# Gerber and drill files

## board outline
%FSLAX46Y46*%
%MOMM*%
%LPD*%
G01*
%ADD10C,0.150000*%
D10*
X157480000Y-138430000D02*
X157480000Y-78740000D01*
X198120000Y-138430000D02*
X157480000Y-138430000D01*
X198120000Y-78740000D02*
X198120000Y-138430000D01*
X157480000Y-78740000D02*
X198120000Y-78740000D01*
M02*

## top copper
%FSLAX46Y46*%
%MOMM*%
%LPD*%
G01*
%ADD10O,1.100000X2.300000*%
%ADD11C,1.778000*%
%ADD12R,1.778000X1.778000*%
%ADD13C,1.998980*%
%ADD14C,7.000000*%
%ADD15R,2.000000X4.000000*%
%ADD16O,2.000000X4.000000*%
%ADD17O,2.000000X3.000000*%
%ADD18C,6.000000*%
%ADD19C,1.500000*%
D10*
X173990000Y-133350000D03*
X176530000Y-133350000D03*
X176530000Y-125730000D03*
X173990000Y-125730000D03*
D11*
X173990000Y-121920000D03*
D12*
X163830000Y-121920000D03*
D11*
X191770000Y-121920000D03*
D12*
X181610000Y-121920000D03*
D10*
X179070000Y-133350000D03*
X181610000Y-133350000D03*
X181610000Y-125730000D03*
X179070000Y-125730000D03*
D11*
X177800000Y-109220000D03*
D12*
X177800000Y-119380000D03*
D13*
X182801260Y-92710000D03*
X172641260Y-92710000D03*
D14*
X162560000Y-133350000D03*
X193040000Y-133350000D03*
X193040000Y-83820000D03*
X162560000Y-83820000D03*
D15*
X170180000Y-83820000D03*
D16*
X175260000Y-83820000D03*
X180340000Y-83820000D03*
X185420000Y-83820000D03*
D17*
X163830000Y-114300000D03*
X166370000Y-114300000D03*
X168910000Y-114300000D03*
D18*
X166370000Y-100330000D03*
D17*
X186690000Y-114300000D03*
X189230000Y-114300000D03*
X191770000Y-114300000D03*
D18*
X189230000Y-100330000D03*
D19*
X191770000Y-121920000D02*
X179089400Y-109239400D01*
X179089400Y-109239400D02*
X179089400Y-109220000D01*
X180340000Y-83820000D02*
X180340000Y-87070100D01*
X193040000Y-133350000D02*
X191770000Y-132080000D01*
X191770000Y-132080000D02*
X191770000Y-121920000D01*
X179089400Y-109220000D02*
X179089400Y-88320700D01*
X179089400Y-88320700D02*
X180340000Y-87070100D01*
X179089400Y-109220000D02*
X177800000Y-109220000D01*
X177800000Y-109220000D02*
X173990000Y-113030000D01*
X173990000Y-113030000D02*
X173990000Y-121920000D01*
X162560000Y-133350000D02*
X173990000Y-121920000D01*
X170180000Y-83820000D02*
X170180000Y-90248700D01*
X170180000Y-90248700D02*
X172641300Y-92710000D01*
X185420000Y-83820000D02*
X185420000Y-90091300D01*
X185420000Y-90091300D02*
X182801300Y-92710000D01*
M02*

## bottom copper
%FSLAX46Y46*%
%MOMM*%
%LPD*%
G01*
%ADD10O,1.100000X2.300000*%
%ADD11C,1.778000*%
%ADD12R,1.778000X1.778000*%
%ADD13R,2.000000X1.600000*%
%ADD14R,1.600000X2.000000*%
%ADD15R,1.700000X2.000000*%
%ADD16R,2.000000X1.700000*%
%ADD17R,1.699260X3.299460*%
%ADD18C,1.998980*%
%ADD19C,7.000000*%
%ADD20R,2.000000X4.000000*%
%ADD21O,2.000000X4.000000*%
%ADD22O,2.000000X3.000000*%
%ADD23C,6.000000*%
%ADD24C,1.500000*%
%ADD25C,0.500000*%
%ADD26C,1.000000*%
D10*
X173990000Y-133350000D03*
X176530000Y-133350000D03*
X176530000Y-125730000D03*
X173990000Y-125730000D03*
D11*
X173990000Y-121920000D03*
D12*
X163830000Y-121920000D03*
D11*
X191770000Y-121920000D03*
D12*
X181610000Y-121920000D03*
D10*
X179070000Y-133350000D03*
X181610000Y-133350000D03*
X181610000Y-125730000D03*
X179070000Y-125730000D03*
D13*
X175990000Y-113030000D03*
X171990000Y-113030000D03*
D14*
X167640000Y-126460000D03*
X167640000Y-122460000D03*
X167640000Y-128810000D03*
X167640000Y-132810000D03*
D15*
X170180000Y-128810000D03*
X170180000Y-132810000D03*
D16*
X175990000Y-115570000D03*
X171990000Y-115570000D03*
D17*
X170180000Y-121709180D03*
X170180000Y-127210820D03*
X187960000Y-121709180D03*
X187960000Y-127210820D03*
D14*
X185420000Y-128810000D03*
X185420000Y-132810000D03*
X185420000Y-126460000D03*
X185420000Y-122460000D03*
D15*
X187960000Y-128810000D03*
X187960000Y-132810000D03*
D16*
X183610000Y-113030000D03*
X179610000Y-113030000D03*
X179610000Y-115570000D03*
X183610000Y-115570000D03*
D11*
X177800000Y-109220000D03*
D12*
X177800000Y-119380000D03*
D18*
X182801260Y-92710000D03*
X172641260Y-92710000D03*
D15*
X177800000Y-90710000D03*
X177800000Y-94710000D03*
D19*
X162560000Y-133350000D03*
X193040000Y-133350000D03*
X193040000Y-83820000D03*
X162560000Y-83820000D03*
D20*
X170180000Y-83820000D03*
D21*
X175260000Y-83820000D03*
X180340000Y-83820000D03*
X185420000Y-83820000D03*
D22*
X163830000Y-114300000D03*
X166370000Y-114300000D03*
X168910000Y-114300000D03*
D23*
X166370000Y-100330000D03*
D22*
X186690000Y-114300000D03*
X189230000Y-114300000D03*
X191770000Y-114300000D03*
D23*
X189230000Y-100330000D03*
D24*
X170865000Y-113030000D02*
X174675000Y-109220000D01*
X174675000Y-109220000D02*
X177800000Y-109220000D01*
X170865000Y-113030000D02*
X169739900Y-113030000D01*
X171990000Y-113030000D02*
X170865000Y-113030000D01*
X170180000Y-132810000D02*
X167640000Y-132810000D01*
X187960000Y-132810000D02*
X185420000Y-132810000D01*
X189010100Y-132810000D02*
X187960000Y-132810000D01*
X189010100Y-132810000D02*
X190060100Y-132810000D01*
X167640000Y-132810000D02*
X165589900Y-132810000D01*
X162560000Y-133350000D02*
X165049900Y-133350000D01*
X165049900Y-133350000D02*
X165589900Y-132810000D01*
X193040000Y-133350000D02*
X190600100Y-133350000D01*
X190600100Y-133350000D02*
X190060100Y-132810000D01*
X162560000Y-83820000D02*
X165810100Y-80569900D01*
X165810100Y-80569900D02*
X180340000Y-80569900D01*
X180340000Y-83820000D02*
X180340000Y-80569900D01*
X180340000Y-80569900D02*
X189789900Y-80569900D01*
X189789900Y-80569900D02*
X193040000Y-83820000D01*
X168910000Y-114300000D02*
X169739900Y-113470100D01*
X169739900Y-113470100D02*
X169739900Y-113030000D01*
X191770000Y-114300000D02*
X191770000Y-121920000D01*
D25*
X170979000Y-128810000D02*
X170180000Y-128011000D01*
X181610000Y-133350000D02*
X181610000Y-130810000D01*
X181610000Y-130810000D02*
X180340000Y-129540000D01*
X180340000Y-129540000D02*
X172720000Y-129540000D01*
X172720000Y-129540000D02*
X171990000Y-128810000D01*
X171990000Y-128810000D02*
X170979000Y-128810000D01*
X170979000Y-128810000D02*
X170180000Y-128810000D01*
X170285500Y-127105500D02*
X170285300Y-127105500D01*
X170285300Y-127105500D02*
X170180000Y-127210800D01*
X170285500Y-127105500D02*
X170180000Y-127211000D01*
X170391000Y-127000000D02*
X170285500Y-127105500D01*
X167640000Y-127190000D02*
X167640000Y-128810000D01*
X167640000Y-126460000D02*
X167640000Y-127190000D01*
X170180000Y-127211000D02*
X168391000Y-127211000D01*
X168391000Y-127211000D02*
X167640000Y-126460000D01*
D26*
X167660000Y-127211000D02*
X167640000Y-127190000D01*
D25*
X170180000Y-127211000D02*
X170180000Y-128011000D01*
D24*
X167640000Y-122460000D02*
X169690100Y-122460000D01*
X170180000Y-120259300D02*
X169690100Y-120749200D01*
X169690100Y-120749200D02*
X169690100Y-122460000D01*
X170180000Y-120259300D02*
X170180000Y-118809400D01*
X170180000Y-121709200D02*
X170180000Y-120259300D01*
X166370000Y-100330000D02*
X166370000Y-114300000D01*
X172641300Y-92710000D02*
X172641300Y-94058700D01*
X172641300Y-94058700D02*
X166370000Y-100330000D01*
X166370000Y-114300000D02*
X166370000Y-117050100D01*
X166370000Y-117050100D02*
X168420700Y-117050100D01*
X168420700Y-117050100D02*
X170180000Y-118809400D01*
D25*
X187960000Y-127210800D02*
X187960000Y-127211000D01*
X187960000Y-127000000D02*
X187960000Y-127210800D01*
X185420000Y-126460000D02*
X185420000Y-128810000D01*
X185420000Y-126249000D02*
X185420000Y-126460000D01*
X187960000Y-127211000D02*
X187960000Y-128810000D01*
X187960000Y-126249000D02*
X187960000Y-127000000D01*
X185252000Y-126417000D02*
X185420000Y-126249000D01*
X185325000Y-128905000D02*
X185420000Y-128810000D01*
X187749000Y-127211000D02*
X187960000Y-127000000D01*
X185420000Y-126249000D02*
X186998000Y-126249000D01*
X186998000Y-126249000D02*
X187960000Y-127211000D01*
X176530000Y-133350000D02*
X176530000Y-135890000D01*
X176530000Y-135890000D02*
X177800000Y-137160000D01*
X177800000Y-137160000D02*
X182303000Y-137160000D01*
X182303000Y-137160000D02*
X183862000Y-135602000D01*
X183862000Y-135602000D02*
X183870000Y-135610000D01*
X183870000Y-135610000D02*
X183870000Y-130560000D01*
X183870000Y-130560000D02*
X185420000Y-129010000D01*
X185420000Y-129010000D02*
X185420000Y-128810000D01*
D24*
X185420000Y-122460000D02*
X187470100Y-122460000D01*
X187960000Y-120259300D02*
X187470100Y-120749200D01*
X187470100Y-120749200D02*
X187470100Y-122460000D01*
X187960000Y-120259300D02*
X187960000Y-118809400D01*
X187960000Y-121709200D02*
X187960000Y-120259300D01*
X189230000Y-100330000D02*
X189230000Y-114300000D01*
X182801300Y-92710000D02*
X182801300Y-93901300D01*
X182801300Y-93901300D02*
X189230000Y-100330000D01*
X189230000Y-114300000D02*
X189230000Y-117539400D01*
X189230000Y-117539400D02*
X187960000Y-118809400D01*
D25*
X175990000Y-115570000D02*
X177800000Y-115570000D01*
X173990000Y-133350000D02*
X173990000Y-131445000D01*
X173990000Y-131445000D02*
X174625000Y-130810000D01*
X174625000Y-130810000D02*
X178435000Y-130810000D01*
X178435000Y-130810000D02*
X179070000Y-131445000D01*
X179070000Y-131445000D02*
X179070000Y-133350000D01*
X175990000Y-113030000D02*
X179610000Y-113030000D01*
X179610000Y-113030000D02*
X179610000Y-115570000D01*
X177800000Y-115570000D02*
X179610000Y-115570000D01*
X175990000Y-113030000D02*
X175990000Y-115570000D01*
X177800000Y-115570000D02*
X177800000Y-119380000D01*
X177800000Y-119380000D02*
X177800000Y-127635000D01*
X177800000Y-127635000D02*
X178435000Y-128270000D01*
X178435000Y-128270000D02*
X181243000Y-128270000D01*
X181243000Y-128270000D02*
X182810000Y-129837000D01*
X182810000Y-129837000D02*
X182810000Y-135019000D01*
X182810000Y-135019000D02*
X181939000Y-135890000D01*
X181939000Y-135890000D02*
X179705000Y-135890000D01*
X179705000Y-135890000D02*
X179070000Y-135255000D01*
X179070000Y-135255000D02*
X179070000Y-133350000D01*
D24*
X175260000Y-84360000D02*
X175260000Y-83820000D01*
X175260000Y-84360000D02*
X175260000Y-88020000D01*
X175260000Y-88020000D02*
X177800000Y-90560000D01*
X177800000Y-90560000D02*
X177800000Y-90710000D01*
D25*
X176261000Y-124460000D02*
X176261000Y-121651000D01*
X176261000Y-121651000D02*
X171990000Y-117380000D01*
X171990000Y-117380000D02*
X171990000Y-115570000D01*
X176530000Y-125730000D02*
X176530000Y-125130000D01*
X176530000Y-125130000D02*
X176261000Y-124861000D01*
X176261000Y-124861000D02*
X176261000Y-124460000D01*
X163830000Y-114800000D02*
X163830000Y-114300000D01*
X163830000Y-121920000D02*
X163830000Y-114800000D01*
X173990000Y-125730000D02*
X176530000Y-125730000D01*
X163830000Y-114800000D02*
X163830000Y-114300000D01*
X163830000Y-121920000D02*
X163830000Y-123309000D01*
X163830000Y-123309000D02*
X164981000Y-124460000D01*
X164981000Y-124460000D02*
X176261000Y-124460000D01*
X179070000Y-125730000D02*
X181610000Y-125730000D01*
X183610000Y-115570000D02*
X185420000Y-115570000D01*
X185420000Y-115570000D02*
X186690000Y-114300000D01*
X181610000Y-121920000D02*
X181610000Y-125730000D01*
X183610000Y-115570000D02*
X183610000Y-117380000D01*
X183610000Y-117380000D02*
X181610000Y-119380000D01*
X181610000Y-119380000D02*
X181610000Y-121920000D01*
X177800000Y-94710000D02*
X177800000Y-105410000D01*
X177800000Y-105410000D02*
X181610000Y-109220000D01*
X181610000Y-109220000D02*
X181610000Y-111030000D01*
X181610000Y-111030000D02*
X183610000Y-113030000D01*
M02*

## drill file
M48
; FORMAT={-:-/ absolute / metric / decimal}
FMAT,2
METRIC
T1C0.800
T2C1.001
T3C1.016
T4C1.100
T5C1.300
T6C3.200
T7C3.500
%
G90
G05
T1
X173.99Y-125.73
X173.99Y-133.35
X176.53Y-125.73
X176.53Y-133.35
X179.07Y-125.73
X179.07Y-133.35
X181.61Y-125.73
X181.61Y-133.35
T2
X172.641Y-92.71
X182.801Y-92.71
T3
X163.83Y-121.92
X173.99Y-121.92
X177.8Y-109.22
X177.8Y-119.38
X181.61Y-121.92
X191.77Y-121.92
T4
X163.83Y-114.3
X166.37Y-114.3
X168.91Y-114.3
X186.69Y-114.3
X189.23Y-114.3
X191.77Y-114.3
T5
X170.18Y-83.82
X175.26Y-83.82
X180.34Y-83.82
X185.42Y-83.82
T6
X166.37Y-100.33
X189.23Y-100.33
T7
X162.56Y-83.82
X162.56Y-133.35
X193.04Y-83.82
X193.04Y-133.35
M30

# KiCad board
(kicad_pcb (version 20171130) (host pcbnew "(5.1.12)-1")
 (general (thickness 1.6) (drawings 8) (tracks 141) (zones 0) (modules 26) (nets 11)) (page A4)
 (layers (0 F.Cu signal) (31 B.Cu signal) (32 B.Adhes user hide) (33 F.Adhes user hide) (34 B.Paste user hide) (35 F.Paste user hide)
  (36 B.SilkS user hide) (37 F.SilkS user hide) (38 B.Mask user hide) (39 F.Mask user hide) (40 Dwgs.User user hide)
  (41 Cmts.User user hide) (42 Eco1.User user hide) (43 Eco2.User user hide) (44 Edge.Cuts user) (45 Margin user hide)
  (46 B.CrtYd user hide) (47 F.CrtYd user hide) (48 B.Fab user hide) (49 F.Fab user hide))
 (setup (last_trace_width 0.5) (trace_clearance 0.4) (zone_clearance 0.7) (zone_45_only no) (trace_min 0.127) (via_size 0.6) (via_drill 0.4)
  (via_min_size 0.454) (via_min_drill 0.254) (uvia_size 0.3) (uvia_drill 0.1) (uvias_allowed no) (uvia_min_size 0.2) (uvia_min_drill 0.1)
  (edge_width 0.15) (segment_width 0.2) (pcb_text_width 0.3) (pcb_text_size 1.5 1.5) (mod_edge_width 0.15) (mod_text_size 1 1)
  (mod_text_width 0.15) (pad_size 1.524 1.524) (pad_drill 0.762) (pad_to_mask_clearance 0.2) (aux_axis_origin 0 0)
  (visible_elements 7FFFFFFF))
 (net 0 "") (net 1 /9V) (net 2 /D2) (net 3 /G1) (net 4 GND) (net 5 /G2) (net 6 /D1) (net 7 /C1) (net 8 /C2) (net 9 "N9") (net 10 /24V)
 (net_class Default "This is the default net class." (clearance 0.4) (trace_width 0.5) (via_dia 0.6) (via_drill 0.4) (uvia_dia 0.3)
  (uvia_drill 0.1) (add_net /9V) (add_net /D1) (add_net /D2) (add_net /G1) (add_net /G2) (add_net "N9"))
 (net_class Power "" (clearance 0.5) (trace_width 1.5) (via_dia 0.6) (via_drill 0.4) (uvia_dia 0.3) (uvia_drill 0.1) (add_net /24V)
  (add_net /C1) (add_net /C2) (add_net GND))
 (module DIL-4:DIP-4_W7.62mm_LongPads (layer F.Cu) (at 173.99 133.35 90)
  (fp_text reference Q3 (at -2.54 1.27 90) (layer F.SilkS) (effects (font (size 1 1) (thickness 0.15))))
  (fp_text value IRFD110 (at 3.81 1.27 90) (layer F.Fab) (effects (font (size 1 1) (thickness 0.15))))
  (pad 1 thru_hole oval (at 0 0 90) (size 2.3 1.1) (drill 0.8) (layers *.Cu *.Mask) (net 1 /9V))
  (pad 2 thru_hole oval (at 0 2.54 90) (size 2.3 1.1) (drill 0.8) (layers *.Cu *.Mask) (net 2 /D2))
  (pad 3 thru_hole oval (at 7.62 2.54 90) (size 2.3 1.1) (drill 0.8) (layers *.Cu *.Mask) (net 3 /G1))
  (pad 3 thru_hole oval (at 7.62 0 90) (size 2.3 1.1) (drill 0.8) (layers *.Cu *.Mask) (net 3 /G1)))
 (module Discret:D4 (layer F.Cu) (at 168.91 121.92 180)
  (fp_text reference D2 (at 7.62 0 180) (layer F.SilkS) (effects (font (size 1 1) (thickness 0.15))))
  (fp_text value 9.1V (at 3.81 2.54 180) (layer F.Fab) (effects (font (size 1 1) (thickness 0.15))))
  (pad 2 thru_hole circle (at -5.08 0 180) (size 1.778 1.778) (drill 1.016) (layers *.Cu *.Mask) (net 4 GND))
  (pad 1 thru_hole rect (at 5.08 0 180) (size 1.778 1.778) (drill 1.016) (layers *.Cu *.Mask) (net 3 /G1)))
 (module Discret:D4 (layer F.Cu) (at 186.69 121.92 180)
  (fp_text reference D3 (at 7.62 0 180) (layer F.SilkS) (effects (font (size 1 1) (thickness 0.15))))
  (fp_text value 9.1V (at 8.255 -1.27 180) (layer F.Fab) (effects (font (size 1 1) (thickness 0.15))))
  (pad 2 thru_hole circle (at -5.08 0 180) (size 1.778 1.778) (drill 1.016) (layers *.Cu *.Mask) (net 4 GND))
  (pad 1 thru_hole rect (at 5.08 0 180) (size 1.778 1.778) (drill 1.016) (layers *.Cu *.Mask) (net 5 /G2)))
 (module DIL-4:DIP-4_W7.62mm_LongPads (layer F.Cu) (at 179.07 133.35 90)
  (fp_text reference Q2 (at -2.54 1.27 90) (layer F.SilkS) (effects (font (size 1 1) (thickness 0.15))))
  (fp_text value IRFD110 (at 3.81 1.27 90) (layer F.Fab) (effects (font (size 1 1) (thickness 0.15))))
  (pad 1 thru_hole oval (at 0 0 90) (size 2.3 1.1) (drill 0.8) (layers *.Cu *.Mask) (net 1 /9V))
  (pad 2 thru_hole oval (at 0 2.54 90) (size 2.3 1.1) (drill 0.8) (layers *.Cu *.Mask) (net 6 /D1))
  (pad 3 thru_hole oval (at 7.62 2.54 90) (size 2.3 1.1) (drill 0.8) (layers *.Cu *.Mask) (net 5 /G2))
  (pad 3 thru_hole oval (at 7.62 0 90) (size 2.3 1.1) (drill 0.8) (layers *.Cu *.Mask) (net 5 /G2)))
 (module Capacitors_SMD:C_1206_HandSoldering (layer B.Cu) (at 173.99 113.03 180)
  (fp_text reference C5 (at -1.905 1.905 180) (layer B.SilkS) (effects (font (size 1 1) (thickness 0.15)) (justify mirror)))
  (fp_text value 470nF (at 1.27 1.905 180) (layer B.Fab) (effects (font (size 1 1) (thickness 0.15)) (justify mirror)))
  (pad 1 smd rect (at -2 0 180) (size 2 1.6) (layers B.Cu B.Paste B.Mask) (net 1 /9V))
  (pad 2 smd rect (at 2 0 180) (size 2 1.6) (layers B.Cu B.Paste B.Mask) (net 4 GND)))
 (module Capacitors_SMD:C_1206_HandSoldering (layer B.Cu) (at 167.64 124.46 90)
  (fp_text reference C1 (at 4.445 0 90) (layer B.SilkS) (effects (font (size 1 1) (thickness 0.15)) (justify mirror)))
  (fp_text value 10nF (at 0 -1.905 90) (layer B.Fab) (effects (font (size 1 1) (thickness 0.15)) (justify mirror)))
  (pad 1 smd rect (at -2 0 90) (size 2 1.6) (layers B.Cu B.Paste B.Mask) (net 6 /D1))
  (pad 2 smd rect (at 2 0 90) (size 2 1.6) (layers B.Cu B.Paste B.Mask) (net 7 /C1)))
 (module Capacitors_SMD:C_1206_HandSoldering (layer B.Cu) (at 167.64 130.81 270)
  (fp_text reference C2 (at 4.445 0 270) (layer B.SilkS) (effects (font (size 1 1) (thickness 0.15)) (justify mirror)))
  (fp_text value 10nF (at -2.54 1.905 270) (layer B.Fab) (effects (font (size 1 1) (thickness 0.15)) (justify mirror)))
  (pad 1 smd rect (at -2 0 270) (size 2 1.6) (layers B.Cu B.Paste B.Mask) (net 6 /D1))
  (pad 2 smd rect (at 2 0 270) (size 2 1.6) (layers B.Cu B.Paste B.Mask) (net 4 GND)))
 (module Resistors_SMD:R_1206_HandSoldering (layer B.Cu) (at 170.18 130.81 270)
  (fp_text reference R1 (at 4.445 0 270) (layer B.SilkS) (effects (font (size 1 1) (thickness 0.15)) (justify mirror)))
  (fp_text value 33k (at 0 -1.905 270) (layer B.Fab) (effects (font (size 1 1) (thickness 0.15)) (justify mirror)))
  (pad 1 smd rect (at -2 0 270) (size 2 1.7) (layers B.Cu B.Paste B.Mask) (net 6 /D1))
  (pad 2 smd rect (at 2 0 270) (size 2 1.7) (layers B.Cu B.Paste B.Mask) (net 4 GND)))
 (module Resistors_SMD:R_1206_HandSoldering (layer B.Cu) (at 173.99 115.57 180)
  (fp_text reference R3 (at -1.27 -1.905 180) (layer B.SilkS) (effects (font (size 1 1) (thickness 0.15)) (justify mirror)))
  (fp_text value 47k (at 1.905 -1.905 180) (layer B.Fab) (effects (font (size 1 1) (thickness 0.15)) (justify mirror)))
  (pad 1 smd rect (at -2 0 180) (size 2 1.7) (layers B.Cu B.Paste B.Mask) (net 1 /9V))
  (pad 2 smd rect (at 2 0 180) (size 2 1.7) (layers B.Cu B.Paste B.Mask) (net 3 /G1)))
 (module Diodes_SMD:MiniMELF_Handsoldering (layer B.Cu) (at 170.18 124.46 270)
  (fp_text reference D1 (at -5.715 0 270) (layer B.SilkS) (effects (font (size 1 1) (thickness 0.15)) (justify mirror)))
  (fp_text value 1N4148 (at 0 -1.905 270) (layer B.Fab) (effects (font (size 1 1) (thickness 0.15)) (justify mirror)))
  (pad 1 smd rect (at -2.75082 0 270) (size 3.29946 1.69926) (layers B.Cu B.Paste B.Mask) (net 7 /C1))
  (pad 2 smd rect (at 2.75082 0 270) (size 3.29946 1.69926) (layers B.Cu B.Paste B.Mask) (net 6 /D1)))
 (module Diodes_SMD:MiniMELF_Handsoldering (layer B.Cu) (at 187.96 124.46 270)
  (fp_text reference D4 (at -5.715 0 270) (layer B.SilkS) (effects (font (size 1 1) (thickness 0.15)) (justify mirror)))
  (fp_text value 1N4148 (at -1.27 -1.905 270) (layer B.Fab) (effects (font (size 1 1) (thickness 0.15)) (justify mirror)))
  (pad 1 smd rect (at -2.75082 0 270) (size 3.29946 1.69926) (layers B.Cu B.Paste B.Mask) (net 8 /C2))
  (pad 2 smd rect (at 2.75082 0 270) (size 3.29946 1.69926) (layers B.Cu B.Paste B.Mask) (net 2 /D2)))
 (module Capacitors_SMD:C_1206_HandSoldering (layer B.Cu) (at 185.42 130.81 270)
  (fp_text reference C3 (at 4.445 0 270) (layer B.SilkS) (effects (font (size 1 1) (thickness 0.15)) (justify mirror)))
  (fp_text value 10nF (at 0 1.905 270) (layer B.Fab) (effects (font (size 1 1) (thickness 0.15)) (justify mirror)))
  (pad 1 smd rect (at -2 0 270) (size 2 1.6) (layers B.Cu B.Paste B.Mask) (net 2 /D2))
  (pad 2 smd rect (at 2 0 270) (size 2 1.6) (layers B.Cu B.Paste B.Mask) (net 4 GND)))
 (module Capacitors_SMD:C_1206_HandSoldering (layer B.Cu) (at 185.42 124.46 90)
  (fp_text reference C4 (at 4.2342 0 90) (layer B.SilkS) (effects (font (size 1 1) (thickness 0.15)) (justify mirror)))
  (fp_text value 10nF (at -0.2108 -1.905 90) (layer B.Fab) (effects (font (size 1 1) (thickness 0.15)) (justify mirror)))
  (pad 1 smd rect (at -2 0 90) (size 2 1.6) (layers B.Cu B.Paste B.Mask) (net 2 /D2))
  (pad 2 smd rect (at 2 0 90) (size 2 1.6) (layers B.Cu B.Paste B.Mask) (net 8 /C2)))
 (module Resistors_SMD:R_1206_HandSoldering (layer B.Cu) (at 187.96 130.81 270)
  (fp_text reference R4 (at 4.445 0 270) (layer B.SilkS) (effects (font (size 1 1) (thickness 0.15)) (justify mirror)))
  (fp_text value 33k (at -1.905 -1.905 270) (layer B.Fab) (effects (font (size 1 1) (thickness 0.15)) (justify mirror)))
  (pad 1 smd rect (at -2 0 270) (size 2 1.7) (layers B.Cu B.Paste B.Mask) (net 2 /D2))
  (pad 2 smd rect (at 2 0 270) (size 2 1.7) (layers B.Cu B.Paste B.Mask) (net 4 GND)))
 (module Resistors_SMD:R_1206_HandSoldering (layer B.Cu) (at 181.61 113.03 180)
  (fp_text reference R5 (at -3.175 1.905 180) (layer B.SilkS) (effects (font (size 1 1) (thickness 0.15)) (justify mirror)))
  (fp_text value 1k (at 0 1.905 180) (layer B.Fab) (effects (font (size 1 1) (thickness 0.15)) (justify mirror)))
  (pad 1 smd rect (at -2 0 180) (size 2 1.7) (layers B.Cu B.Paste B.Mask) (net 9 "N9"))
  (pad 2 smd rect (at 2 0 180) (size 2 1.7) (layers B.Cu B.Paste B.Mask) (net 1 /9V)))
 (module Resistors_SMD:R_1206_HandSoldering (layer B.Cu) (at 181.61 115.57)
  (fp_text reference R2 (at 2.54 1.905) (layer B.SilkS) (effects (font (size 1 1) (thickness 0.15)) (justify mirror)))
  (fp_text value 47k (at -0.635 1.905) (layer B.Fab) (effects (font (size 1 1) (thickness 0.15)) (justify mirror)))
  (pad 1 smd rect (at -2 0) (size 2 1.7) (layers B.Cu B.Paste B.Mask) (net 1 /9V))
  (pad 2 smd rect (at 2 0) (size 2 1.7) (layers B.Cu B.Paste B.Mask) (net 5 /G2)))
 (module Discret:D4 (layer F.Cu) (at 177.8 114.3 270)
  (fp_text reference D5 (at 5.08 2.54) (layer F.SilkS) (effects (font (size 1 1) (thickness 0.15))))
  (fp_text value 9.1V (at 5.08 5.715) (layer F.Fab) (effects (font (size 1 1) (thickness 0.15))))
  (pad 2 thru_hole circle (at -5.08 0 270) (size 1.778 1.778) (drill 1.016) (layers *.Cu *.Mask) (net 4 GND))
  (pad 1 thru_hole rect (at 5.08 0 270) (size 1.778 1.778) (drill 1.016) (layers *.Cu *.Mask) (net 1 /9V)))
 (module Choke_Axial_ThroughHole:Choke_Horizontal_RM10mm (layer F.Cu) (at 177.8 92.71 180)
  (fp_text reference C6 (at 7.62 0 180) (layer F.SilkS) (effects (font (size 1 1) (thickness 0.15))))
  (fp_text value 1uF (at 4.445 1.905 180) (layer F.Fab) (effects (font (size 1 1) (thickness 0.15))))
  (pad 1 thru_hole circle (at -5.00126 0 180) (size 1.99898 1.99898) (drill 1.00076) (layers *.Cu *.Mask) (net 8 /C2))
  (pad 2 thru_hole circle (at 5.15874 0 180) (size 1.99898 1.99898) (drill 1.00076) (layers *.Cu *.Mask) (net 7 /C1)))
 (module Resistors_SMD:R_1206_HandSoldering (layer B.Cu) (at 177.8 92.71 270)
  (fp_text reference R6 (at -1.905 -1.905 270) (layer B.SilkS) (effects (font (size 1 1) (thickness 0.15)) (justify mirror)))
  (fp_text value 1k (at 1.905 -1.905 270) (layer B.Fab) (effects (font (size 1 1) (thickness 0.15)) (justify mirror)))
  (pad 1 smd rect (at -2 0 270) (size 2 1.7) (layers B.Cu B.Paste B.Mask) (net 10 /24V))
  (pad 2 smd rect (at 2 0 270) (size 2 1.7) (layers B.Cu B.Paste B.Mask) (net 9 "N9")))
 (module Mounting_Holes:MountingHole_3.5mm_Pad (layer F.Cu) (at 162.56 133.35)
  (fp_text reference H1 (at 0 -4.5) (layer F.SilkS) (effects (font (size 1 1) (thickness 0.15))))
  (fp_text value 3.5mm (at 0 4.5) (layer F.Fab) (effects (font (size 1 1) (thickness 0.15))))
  (pad 1 thru_hole circle (at 0 0) (size 7 7) (drill 3.5) (layers *.Cu *.Mask) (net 4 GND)))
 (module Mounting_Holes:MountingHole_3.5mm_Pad (layer F.Cu) (at 193.04 133.35)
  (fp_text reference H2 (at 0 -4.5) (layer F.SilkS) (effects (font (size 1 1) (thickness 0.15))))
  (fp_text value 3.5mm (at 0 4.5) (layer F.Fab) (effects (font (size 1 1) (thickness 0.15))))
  (pad 1 thru_hole circle (at 0 0) (size 7 7) (drill 3.5) (layers *.Cu *.Mask) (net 4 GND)))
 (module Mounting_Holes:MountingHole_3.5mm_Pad (layer F.Cu) (at 193.04 83.82)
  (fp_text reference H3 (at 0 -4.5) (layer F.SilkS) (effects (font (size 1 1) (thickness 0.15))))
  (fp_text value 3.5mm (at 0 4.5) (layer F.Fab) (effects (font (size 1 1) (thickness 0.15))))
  (pad 1 thru_hole circle (at 0 0) (size 7 7) (drill 3.5) (layers *.Cu *.Mask) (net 4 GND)))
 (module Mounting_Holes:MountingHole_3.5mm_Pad (layer F.Cu) (at 162.56 83.82)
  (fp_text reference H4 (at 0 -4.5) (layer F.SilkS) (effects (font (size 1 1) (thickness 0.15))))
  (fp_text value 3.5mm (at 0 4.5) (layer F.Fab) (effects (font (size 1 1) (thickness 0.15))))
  (pad 1 thru_hole circle (at 0 0) (size 7 7) (drill 3.5) (layers *.Cu *.Mask) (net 4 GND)))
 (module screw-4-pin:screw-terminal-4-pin (layer F.Cu) (at 170.18 83.82)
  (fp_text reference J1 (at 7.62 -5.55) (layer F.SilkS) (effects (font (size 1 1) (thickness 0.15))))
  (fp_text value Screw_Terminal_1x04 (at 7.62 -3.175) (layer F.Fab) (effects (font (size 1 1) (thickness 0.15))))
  (pad 1 thru_hole rect (at 0 0) (size 2 4) (drill 1.3) (layers *.Cu *.Mask) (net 7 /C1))
  (pad 2 thru_hole oval (at 5.08 0) (size 2 4) (drill 1.3) (layers *.Cu *.Mask) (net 10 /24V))
  (pad 3 thru_hole oval (at 10.16 0) (size 2 4) (drill 1.3) (layers *.Cu *.Mask) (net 4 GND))
  (pad 4 thru_hole oval (at 15.24 0) (size 2 4) (drill 1.3) (layers *.Cu *.Mask) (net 8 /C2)))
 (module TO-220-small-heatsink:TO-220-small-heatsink (layer F.Cu) (at 166.37 114.3)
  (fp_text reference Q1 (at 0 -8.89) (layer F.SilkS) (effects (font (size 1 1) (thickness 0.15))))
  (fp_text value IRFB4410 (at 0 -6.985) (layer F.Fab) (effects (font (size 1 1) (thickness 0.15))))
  (pad 1 thru_hole oval (at -2.54 0) (size 2 3) (drill 1.1) (layers B.Cu B.Mask) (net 3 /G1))
  (pad 2 thru_hole oval (at 0 0) (size 2 3) (drill 1.1) (layers B.Cu B.Mask) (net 7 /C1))
  (pad 3 thru_hole oval (at 2.54 0) (size 2 3) (drill 1.1) (layers B.Cu B.Mask) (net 4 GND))
  (pad 2 thru_hole circle (at 0 -13.97) (size 6 6) (drill 3.2) (layers B.Cu B.Mask) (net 7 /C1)))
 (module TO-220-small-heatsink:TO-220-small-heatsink (layer F.Cu) (at 189.23 114.3)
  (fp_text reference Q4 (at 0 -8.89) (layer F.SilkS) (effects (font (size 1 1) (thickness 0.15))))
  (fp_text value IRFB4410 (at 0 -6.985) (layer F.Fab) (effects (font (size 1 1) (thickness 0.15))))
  (pad 1 thru_hole oval (at -2.54 0) (size 2 3) (drill 1.1) (layers B.Cu B.Mask) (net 5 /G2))
  (pad 2 thru_hole oval (at 0 0) (size 2 3) (drill 1.1) (layers B.Cu B.Mask) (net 8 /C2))
  (pad 3 thru_hole oval (at 2.54 0) (size 2 3) (drill 1.1) (layers B.Cu B.Mask) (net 4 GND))
  (pad 2 thru_hole circle (at 0 -13.97) (size 6 6) (drill 3.2) (layers B.Cu B.Mask) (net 8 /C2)))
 (gr_line (start 157.48 138.43) (end 157.48 78.74) (angle 90) (layer Edge.Cuts) (width 0.15))
 (gr_line (start 198.12 138.43) (end 157.48 138.43) (angle 90) (layer Edge.Cuts) (width 0.15))
 (gr_line (start 198.12 78.74) (end 198.12 138.43) (angle 90) (layer Edge.Cuts) (width 0.15))
 (gr_line (start 157.48 78.74) (end 198.12 78.74) (angle 90) (layer Edge.Cuts) (width 0.15))
 (segment (start 191.77 121.92) (end 179.0894 109.2394) (width 1.5) (layer F.Cu) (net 4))
 (segment (start 179.0894 109.2394) (end 179.0894 109.22) (width 1.5) (layer F.Cu) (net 4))
 (segment (start 180.34 83.82) (end 180.34 87.0701) (width 1.5) (layer F.Cu) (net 4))
 (segment (start 193.04 133.35) (end 191.77 132.08) (width 1.5) (layer F.Cu) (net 4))
 (segment (start 191.77 132.08) (end 191.77 121.92) (width 1.5) (layer F.Cu) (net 4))
 (segment (start 179.0894 109.22) (end 179.0894 88.3207) (width 1.5) (layer F.Cu) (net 4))
 (segment (start 179.0894 88.3207) (end 180.34 87.0701) (width 1.5) (layer F.Cu) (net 4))
 (segment (start 179.0894 109.22) (end 177.8 109.22) (width 1.5) (layer F.Cu) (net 4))
 (segment (start 177.8 109.22) (end 173.99 113.03) (width 1.5) (layer F.Cu) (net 4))
 (segment (start 173.99 113.03) (end 173.99 121.92) (width 1.5) (layer F.Cu) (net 4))
 (segment (start 170.865 113.03) (end 174.675 109.22) (width 1.5) (layer B.Cu) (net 4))
 (segment (start 174.675 109.22) (end 177.8 109.22) (width 1.5) (layer B.Cu) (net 4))
 (segment (start 170.865 113.03) (end 169.7399 113.03) (width 1.5) (layer B.Cu) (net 4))
 (segment (start 171.99 113.03) (end 170.865 113.03) (width 1.5) (layer B.Cu) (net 4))
 (segment (start 162.56 133.35) (end 173.99 121.92) (width 1.5) (layer F.Cu) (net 4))
 (segment (start 170.18 132.81) (end 167.64 132.81) (width 1.5) (layer B.Cu) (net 4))
 (segment (start 187.96 132.81) (end 185.42 132.81) (width 1.5) (layer B.Cu) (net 4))
 (segment (start 189.0101 132.81) (end 187.96 132.81) (width 1.5) (layer B.Cu) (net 4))
 (segment (start 189.0101 132.81) (end 190.0601 132.81) (width 1.5) (layer B.Cu) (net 4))
 (segment (start 167.64 132.81) (end 165.5899 132.81) (width 1.5) (layer B.Cu) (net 4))
 (segment (start 162.56 133.35) (end 165.0499 133.35) (width 1.5) (layer B.Cu) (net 4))
 (segment (start 165.0499 133.35) (end 165.5899 132.81) (width 1.5) (layer B.Cu) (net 4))
 (segment (start 193.04 133.35) (end 190.6001 133.35) (width 1.5) (layer B.Cu) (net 4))
 (segment (start 190.6001 133.35) (end 190.0601 132.81) (width 1.5) (layer B.Cu) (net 4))
 (segment (start 162.56 83.82) (end 165.8101 80.5699) (width 1.5) (layer B.Cu) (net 4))
 (segment (start 165.8101 80.5699) (end 180.34 80.5699) (width 1.5) (layer B.Cu) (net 4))
 (segment (start 180.34 83.82) (end 180.34 80.5699) (width 1.5) (layer B.Cu) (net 4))
 (segment (start 180.34 80.5699) (end 189.7899 80.5699) (width 1.5) (layer B.Cu) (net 4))
 (segment (start 189.7899 80.5699) (end 193.04 83.82) (width 1.5) (layer B.Cu) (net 4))
 (segment (start 168.91 114.3) (end 169.7399 113.4701) (width 1.5) (layer B.Cu) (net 4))
 (segment (start 169.7399 113.4701) (end 169.7399 113.03) (width 1.5) (layer B.Cu) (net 4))
 (segment (start 191.77 114.3) (end 191.77 121.92) (width 1.5) (layer B.Cu) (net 4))
 (segment (start 170.979 128.81) (end 170.18 128.011) (width 0.5) (layer B.Cu) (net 6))
 (segment (start 181.61 133.35) (end 181.61 130.81) (width 0.5) (layer B.Cu) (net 6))
 (segment (start 181.61 130.81) (end 180.34 129.54) (width 0.5) (layer B.Cu) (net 6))
 (segment (start 180.34 129.54) (end 172.72 129.54) (width 0.5) (layer B.Cu) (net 6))
 (segment (start 172.72 129.54) (end 171.99 128.81) (width 0.5) (layer B.Cu) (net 6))
 (segment (start 171.99 128.81) (end 170.979 128.81) (width 0.5) (layer B.Cu) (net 6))
 (segment (start 170.979 128.81) (end 170.18 128.81) (width 0.5) (layer B.Cu) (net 6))
 (segment (start 170.2855 127.1055) (end 170.2853 127.1055) (width 0.5) (layer B.Cu) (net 6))
 (segment (start 170.2853 127.1055) (end 170.18 127.2108) (width 0.5) (layer B.Cu) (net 6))
 (segment (start 170.2855 127.1055) (end 170.18 127.211) (width 0.5) (layer B.Cu) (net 6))
 (segment (start 170.391 127) (end 170.2855 127.1055) (width 0.5) (layer B.Cu) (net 6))
 (segment (start 167.64 127.19) (end 167.64 128.81) (width 0.5) (layer B.Cu) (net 6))
 (segment (start 167.64 126.46) (end 167.64 127.19) (width 0.5) (layer B.Cu) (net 6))
 (segment (start 170.18 127.211) (end 168.391 127.211) (width 0.5) (layer B.Cu) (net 6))
 (segment (start 168.391 127.211) (end 167.64 126.46) (width 0.5) (layer B.Cu) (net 6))
 (segment (start 167.66 127.211) (end 167.64 127.19) (width 1) (layer B.Cu) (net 6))
 (segment (start 170.18 127.211) (end 170.18 128.011) (width 0.5) (layer B.Cu) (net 6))
 (segment (start 167.64 122.46) (end 169.6901 122.46) (width 1.5) (layer B.Cu) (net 7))
 (segment (start 170.18 120.2593) (end 169.6901 120.7492) (width 1.5) (layer B.Cu) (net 7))
 (segment (start 169.6901 120.7492) (end 169.6901 122.46) (width 1.5) (layer B.Cu) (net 7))
 (segment (start 170.18 120.2593) (end 170.18 118.8094) (width 1.5) (layer B.Cu) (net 7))
 (segment (start 170.18 121.7092) (end 170.18 120.2593) (width 1.5) (layer B.Cu) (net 7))
 (segment (start 166.37 100.33) (end 166.37 114.3) (width 1.5) (layer B.Cu) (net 7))
 (segment (start 172.6413 92.71) (end 172.6413 94.0587) (width 1.5) (layer B.Cu) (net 7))
 (segment (start 172.6413 94.0587) (end 166.37 100.33) (width 1.5) (layer B.Cu) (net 7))
 (segment (start 170.18 83.82) (end 170.18 90.2487) (width 1.5) (layer F.Cu) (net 7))
 (segment (start 170.18 90.2487) (end 172.6413 92.71) (width 1.5) (layer F.Cu) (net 7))
 (segment (start 166.37 114.3) (end 166.37 117.0501) (width 1.5) (layer B.Cu) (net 7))
 (segment (start 166.37 117.0501) (end 168.4207 117.0501) (width 1.5) (layer B.Cu) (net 7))
 (segment (start 168.4207 117.0501) (end 170.18 118.8094) (width 1.5) (layer B.Cu) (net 7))
 (segment (start 187.96 127.2108) (end 187.96 127.211) (width 0.5) (layer B.Cu) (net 2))
 (segment (start 187.96 127) (end 187.96 127.2108) (width 0.5) (layer B.Cu) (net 2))
 (segment (start 185.42 126.46) (end 185.42 128.81) (width 0.5) (layer B.Cu) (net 2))
 (segment (start 185.42 126.249) (end 185.42 126.46) (width 0.5) (layer B.Cu) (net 2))
 (segment (start 187.96 127.211) (end 187.96 128.81) (width 0.5) (layer B.Cu) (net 2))
 (segment (start 187.96 126.249) (end 187.96 127) (width 0.5) (layer B.Cu) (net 2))
 (segment (start 185.252 126.417) (end 185.42 126.249) (width 0.5) (layer B.Cu) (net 2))
 (segment (start 185.325 128.905) (end 185.42 128.81) (width 0.5) (layer B.Cu) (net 2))
 (segment (start 187.749 127.211) (end 187.96 127) (width 0.5) (layer B.Cu) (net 2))
 (segment (start 185.42 126.249) (end 186.998 126.249) (width 0.5) (layer B.Cu) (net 2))
 (segment (start 186.998 126.249) (end 187.96 127.211) (width 0.5) (layer B.Cu) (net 2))
 (segment (start 176.53 133.35) (end 176.53 135.89) (width 0.5) (layer B.Cu) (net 2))
 (segment (start 176.53 135.89) (end 177.8 137.16) (width 0.5) (layer B.Cu) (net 2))
 (segment (start 177.8 137.16) (end 182.303 137.16) (width 0.5) (layer B.Cu) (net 2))
 (segment (start 182.303 137.16) (end 183.862 135.602) (width 0.5) (layer B.Cu) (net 2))
 (segment (start 183.862 135.602) (end 183.87 135.61) (width 0.5) (layer B.Cu) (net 2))
 (segment (start 183.87 135.61) (end 183.87 130.56) (width 0.5) (layer B.Cu) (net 2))
 (segment (start 183.87 130.56) (end 185.42 129.01) (width 0.5) (layer B.Cu) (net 2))
 (segment (start 185.42 129.01) (end 185.42 128.81) (width 0.5) (layer B.Cu) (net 2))
 (segment (start 185.42 122.46) (end 187.4701 122.46) (width 1.5) (layer B.Cu) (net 8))
 (segment (start 187.96 120.2593) (end 187.4701 120.7492) (width 1.5) (layer B.Cu) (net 8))
 (segment (start 187.4701 120.7492) (end 187.4701 122.46) (width 1.5) (layer B.Cu) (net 8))
 (segment (start 187.96 120.2593) (end 187.96 118.8094) (width 1.5) (layer B.Cu) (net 8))
 (segment (start 187.96 121.7092) (end 187.96 120.2593) (width 1.5) (layer B.Cu) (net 8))
 (segment (start 189.23 100.33) (end 189.23 114.3) (width 1.5) (layer B.Cu) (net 8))
 (segment (start 182.8013 92.71) (end 182.8013 93.9013) (width 1.5) (layer B.Cu) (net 8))
 (segment (start 182.8013 93.9013) (end 189.23 100.33) (width 1.5) (layer B.Cu) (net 8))
 (segment (start 185.42 83.82) (end 185.42 90.0913) (width 1.5) (layer F.Cu) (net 8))
 (segment (start 185.42 90.0913) (end 182.8013 92.71) (width 1.5) (layer F.Cu) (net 8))
 (segment (start 189.23 114.3) (end 189.23 117.5394) (width 1.5) (layer B.Cu) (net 8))
 (segment (start 189.23 117.5394) (end 187.96 118.8094) (width 1.5) (layer B.Cu) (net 8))
 (segment (start 175.99 115.57) (end 177.8 115.57) (width 0.5) (layer B.Cu) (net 1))
 (segment (start 173.99 133.35) (end 173.99 131.445) (width 0.5) (layer B.Cu) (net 1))
 (segment (start 173.99 131.445) (end 174.625 130.81) (width 0.5) (layer B.Cu) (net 1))
 (segment (start 174.625 130.81) (end 178.435 130.81) (width 0.5) (layer B.Cu) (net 1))
 (segment (start 178.435 130.81) (end 179.07 131.445) (width 0.5) (layer B.Cu) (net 1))
 (segment (start 179.07 131.445) (end 179.07 133.35) (width 0.5) (layer B.Cu) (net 1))
 (segment (start 175.99 113.03) (end 179.61 113.03) (width 0.5) (layer B.Cu) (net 1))
 (segment (start 179.61 113.03) (end 179.61 115.57) (width 0.5) (layer B.Cu) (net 1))
 (segment (start 177.8 115.57) (end 179.61 115.57) (width 0.5) (layer B.Cu) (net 1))
 (segment (start 175.99 113.03) (end 175.99 115.57) (width 0.5) (layer B.Cu) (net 1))
 (segment (start 177.8 115.57) (end 177.8 119.38) (width 0.5) (layer B.Cu) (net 1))
 (segment (start 177.8 119.38) (end 177.8 127.635) (width 0.5) (layer B.Cu) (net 1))
 (segment (start 177.8 127.635) (end 178.435 128.27) (width 0.5) (layer B.Cu) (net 1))
 (segment (start 178.435 128.27) (end 181.243 128.27) (width 0.5) (layer B.Cu) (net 1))
 (segment (start 181.243 128.27) (end 182.81 129.837) (width 0.5) (layer B.Cu) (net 1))
 (segment (start 182.81 129.837) (end 182.81 135.019) (width 0.5) (layer B.Cu) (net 1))
 (segment (start 182.81 135.019) (end 181.939 135.89) (width 0.5) (layer B.Cu) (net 1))
 (segment (start 181.939 135.89) (end 179.705 135.89) (width 0.5) (layer B.Cu) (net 1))
 (segment (start 179.705 135.89) (end 179.07 135.255) (width 0.5) (layer B.Cu) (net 1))
 (segment (start 179.07 135.255) (end 179.07 133.35) (width 0.5) (layer B.Cu) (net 1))
 (segment (start 175.26 84.36) (end 175.26 83.82) (width 1.5) (layer B.Cu) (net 10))
 (segment (start 175.26 84.36) (end 175.26 88.02) (width 1.5) (layer B.Cu) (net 10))
 (segment (start 175.26 88.02) (end 177.8 90.56) (width 1.5) (layer B.Cu) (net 10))
 (segment (start 177.8 90.56) (end 177.8 90.71) (width 1.5) (layer B.Cu) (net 10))
 (segment (start 176.261 124.46) (end 176.261 121.651) (width 0.5) (layer B.Cu) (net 3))
 (segment (start 176.261 121.651) (end 171.99 117.38) (width 0.5) (layer B.Cu) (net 3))
 (segment (start 171.99 117.38) (end 171.99 115.57) (width 0.5) (layer B.Cu) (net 3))
 (segment (start 176.53 125.73) (end 176.53 125.13) (width 0.5) (layer B.Cu) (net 3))
 (segment (start 176.53 125.13) (end 176.261 124.861) (width 0.5) (layer B.Cu) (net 3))
 (segment (start 176.261 124.861) (end 176.261 124.46) (width 0.5) (layer B.Cu) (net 3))
 (segment (start 163.83 114.8) (end 163.83 114.3) (width 0.5) (layer B.Cu) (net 3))
 (segment (start 163.83 121.92) (end 163.83 114.8) (width 0.5) (layer B.Cu) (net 3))
 (segment (start 173.99 125.73) (end 176.53 125.73) (width 0.5) (layer B.Cu) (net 3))
 (segment (start 163.83 114.8) (end 163.83 114.3) (width 0.5) (layer B.Cu) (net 3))
 (segment (start 163.83 121.92) (end 163.83 123.309) (width 0.5) (layer B.Cu) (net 3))
 (segment (start 163.83 123.309) (end 164.981 124.46) (width 0.5) (layer B.Cu) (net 3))
 (segment (start 164.981 124.46) (end 176.261 124.46) (width 0.5) (layer B.Cu) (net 3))
 (segment (start 179.07 125.73) (end 181.61 125.73) (width 0.5) (layer B.Cu) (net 5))
 (segment (start 183.61 115.57) (end 185.42 115.57) (width 0.5) (layer B.Cu) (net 5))
 (segment (start 185.42 115.57) (end 186.69 114.3) (width 0.5) (layer B.Cu) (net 5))
 (segment (start 181.61 121.92) (end 181.61 125.73) (width 0.5) (layer B.Cu) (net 5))
 (segment (start 183.61 115.57) (end 183.61 117.38) (width 0.5) (layer B.Cu) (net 5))
 (segment (start 183.61 117.38) (end 181.61 119.38) (width 0.5) (layer B.Cu) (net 5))
 (segment (start 181.61 119.38) (end 181.61 121.92) (width 0.5) (layer B.Cu) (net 5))
 (segment (start 177.8 94.71) (end 177.8 105.41) (width 0.5) (layer B.Cu) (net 9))
 (segment (start 177.8 105.41) (end 181.61 109.22) (width 0.5) (layer B.Cu) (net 9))
 (segment (start 181.61 109.22) (end 181.61 111.03) (width 0.5) (layer B.Cu) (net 9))
 (segment (start 181.61 111.03) (end 183.61 113.03) (width 0.5) (layer B.Cu) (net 9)))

